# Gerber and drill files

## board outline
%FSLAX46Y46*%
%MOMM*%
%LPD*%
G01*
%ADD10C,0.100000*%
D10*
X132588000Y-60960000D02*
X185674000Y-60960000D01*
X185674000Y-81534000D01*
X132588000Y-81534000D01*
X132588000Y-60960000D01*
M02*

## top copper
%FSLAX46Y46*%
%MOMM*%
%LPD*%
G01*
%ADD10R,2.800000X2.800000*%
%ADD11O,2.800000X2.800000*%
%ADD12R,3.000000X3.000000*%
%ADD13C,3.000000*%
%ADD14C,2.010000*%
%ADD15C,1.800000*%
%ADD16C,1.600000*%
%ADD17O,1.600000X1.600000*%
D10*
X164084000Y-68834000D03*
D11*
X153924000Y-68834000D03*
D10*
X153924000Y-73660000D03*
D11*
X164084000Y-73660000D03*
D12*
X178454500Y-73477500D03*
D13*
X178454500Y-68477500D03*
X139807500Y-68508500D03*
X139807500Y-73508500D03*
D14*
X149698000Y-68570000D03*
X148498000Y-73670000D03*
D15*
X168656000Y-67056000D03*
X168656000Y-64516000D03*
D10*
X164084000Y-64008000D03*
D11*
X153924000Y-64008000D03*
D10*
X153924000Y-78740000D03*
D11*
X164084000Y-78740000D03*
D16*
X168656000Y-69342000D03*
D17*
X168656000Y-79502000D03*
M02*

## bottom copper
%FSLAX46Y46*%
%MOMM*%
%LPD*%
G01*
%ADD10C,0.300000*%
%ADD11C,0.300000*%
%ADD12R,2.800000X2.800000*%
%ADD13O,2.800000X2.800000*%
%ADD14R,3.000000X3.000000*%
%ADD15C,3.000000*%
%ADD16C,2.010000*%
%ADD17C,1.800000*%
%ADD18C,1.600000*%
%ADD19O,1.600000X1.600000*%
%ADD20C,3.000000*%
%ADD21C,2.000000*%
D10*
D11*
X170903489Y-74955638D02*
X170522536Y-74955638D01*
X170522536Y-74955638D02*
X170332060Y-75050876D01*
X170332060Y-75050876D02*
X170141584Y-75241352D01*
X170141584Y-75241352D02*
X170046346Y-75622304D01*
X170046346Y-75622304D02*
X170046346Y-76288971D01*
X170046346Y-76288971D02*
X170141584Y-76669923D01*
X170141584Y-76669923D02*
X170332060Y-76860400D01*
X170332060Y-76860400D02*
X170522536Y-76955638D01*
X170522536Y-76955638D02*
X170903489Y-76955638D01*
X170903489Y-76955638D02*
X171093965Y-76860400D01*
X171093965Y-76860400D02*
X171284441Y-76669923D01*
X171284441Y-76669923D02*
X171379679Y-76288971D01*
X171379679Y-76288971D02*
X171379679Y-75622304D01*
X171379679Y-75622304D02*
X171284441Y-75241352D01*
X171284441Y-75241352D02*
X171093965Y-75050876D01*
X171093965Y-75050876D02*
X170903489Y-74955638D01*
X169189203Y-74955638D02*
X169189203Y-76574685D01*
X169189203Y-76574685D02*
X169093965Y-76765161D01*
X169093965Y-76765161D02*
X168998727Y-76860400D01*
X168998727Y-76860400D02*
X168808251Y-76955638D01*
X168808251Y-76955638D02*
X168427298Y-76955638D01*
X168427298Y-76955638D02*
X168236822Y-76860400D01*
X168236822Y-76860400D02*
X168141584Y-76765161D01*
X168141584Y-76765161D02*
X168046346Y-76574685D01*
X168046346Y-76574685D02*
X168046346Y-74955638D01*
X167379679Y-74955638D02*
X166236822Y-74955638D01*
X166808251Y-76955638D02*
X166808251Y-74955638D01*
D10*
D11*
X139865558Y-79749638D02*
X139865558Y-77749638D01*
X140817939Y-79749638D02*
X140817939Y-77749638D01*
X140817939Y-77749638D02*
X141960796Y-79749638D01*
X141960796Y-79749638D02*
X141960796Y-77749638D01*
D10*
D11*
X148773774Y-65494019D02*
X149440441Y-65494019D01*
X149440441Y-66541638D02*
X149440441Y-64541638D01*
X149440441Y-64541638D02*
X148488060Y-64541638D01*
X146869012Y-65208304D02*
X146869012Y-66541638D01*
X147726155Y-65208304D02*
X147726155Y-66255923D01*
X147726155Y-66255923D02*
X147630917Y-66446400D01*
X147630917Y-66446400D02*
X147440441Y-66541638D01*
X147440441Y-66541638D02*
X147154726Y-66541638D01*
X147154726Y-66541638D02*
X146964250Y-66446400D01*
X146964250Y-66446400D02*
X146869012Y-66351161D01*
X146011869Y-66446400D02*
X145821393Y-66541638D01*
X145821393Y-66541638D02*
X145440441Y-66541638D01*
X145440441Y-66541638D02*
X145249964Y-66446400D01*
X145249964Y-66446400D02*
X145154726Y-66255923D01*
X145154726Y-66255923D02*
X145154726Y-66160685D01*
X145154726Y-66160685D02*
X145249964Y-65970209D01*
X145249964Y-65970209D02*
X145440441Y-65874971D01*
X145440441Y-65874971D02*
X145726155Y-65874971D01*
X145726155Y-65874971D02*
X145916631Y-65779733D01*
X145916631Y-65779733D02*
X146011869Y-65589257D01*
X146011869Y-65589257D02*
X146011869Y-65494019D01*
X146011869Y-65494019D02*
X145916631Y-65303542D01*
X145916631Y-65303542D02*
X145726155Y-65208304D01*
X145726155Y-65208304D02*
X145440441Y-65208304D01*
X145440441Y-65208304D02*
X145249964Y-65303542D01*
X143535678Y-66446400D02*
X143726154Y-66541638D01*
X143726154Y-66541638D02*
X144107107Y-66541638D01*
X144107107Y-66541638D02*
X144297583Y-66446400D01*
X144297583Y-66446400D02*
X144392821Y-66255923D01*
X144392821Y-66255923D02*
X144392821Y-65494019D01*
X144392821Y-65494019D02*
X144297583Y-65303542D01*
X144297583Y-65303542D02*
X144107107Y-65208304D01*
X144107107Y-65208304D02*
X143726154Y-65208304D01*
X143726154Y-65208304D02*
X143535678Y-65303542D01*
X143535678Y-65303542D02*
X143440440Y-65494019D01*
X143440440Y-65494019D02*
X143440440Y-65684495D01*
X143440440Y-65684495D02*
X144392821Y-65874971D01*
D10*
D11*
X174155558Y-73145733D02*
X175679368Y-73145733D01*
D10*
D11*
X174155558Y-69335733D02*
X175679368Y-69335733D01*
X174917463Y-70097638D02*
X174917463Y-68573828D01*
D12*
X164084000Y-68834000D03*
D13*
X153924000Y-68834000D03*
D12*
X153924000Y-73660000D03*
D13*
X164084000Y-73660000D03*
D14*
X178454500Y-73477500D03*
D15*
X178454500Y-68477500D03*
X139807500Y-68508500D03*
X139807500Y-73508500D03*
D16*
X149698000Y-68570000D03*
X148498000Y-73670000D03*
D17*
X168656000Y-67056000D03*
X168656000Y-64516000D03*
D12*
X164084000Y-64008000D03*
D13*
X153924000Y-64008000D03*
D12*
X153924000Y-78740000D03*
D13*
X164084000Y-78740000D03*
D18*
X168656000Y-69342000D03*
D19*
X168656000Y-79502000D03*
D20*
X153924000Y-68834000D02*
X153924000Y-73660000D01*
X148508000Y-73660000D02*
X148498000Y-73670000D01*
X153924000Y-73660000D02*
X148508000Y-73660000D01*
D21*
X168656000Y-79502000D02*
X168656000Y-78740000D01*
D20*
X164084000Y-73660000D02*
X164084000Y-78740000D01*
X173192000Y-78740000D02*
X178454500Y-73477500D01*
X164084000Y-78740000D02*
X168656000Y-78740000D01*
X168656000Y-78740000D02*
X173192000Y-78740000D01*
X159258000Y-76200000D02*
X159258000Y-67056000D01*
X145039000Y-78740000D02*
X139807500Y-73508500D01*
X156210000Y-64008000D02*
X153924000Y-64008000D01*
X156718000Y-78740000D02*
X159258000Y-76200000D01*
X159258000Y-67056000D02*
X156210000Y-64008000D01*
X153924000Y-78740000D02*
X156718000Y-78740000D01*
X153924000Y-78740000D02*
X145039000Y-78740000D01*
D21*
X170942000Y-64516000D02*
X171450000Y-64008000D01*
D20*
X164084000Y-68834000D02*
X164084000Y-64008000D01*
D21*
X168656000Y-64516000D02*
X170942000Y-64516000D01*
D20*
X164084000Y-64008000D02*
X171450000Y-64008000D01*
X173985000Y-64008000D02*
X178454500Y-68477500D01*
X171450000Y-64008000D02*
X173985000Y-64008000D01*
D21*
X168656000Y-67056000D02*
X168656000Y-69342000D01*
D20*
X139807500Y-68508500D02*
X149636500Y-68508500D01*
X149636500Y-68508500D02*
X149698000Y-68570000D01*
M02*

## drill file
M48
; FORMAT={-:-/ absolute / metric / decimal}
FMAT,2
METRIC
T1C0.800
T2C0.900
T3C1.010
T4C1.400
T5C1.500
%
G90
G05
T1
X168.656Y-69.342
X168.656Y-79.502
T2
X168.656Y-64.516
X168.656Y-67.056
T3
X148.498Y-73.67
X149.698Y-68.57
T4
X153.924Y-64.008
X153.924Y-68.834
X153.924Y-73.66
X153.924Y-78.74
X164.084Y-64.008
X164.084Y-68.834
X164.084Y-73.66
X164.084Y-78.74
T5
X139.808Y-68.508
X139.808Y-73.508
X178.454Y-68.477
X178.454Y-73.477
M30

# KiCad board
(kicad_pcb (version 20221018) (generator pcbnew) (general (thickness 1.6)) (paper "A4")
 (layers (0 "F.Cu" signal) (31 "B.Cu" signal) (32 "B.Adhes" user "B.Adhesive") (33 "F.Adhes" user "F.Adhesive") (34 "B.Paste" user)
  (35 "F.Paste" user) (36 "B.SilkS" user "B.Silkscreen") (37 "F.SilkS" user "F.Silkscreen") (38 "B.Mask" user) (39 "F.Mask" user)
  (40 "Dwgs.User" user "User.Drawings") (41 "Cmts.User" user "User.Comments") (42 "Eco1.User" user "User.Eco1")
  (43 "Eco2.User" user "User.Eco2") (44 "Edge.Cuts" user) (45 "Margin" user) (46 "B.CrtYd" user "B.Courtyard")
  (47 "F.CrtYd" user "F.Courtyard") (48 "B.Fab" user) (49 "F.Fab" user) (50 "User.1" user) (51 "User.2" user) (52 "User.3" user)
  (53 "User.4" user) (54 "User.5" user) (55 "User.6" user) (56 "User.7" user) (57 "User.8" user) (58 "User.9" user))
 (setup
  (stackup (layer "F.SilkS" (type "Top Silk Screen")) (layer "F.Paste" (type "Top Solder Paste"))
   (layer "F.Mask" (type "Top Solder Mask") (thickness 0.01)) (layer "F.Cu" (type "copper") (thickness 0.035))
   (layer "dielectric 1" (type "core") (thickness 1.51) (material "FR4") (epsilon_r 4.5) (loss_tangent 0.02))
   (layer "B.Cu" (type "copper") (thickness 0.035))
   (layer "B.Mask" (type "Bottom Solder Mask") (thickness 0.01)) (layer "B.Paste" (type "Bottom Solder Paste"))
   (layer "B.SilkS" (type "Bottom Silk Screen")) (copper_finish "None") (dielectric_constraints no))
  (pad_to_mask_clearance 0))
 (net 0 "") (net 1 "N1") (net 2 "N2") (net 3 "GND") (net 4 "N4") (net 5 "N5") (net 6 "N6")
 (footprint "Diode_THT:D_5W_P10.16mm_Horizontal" (layer "F.Cu") (at 164.084 68.834 180)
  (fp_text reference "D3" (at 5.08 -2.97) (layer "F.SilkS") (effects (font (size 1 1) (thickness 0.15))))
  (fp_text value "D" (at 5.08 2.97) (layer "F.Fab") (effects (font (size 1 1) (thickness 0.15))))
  (pad "1" thru_hole rect (at 0 0 180) (size 2.8 2.8) (drill 1.4) (layers "*.Cu" "*.Mask") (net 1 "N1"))
  (pad "2" thru_hole oval (at 10.16 0 180) (size 2.8 2.8) (drill 1.4) (layers "*.Cu" "*.Mask") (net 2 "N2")))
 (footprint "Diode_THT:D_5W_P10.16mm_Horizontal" (layer "F.Cu") (at 153.924 73.66)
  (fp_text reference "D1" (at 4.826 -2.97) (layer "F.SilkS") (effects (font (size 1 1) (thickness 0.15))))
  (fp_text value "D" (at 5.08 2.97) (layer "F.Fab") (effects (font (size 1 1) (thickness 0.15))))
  (pad "1" thru_hole rect (at 0 0) (size 2.8 2.8) (drill 1.4) (layers "*.Cu" "*.Mask") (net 2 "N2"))
  (pad "2" thru_hole oval (at 10.16 0) (size 2.8 2.8) (drill 1.4) (layers "*.Cu" "*.Mask") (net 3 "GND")))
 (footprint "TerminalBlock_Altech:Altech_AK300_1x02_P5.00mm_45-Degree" (layer "F.Cu") (at 178.4545 73.4775 90)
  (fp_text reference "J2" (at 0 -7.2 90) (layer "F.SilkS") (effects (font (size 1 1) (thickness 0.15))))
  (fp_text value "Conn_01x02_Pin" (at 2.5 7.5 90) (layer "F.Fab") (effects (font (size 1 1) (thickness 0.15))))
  (pad "1" thru_hole rect (at 0 0 90) (size 3 3) (drill 1.5) (layers "*.Cu" "*.Mask") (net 3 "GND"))
  (pad "2" thru_hole circle (at 5 0 90) (size 3 3) (drill 1.5) (layers "*.Cu" "*.Mask") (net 1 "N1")))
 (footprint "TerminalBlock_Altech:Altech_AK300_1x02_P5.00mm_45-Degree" (layer "F.Cu") (at 139.8075 68.5085 -90)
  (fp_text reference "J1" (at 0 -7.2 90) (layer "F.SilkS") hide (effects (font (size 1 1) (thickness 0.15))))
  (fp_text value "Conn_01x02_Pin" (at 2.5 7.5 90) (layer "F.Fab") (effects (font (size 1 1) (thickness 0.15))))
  (pad "1" thru_hole circle (at 0 0 270) (size 3 3) (drill 1.5) (layers "*.Cu" "*.Mask") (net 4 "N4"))
  (pad "2" thru_hole circle (at 5 0 270) (size 3 3) (drill 1.5) (layers "*.Cu" "*.Mask") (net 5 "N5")))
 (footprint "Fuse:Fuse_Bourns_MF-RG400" (layer "F.Cu") (at 149.698 68.57 -90)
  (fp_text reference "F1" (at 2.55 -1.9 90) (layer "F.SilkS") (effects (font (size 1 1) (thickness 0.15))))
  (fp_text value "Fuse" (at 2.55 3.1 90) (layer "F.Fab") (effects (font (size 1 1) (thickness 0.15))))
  (pad "1" thru_hole circle (at 0 0 270) (size 2.01 2.01) (drill 1.01) (layers "*.Cu" "*.Mask") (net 4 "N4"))
  (pad "2" thru_hole circle (at 5.1 1.2 270) (size 2.01 2.01) (drill 1.01) (layers "*.Cu" "*.Mask") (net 2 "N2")))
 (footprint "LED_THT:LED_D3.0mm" (layer "F.Cu") (at 168.656 67.056 90)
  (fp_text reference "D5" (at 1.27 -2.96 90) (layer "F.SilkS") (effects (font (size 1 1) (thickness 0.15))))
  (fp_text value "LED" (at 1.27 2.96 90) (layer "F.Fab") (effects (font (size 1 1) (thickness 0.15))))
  (pad "1" thru_hole circle (at 0 0 90) (size 1.8 1.8) (drill 0.9) (layers "*.Cu" "*.Mask") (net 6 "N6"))
  (pad "2" thru_hole circle (at 2.54 0 90) (size 1.8 1.8) (drill 0.9) (layers "*.Cu" "*.Mask") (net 1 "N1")))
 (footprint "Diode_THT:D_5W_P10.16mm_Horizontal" (layer "F.Cu") (at 164.084 64.008 180)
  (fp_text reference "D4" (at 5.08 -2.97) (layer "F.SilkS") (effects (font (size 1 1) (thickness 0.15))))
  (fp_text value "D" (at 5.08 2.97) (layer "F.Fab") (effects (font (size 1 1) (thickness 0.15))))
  (pad "1" thru_hole rect (at 0 0 180) (size 2.8 2.8) (drill 1.4) (layers "*.Cu" "*.Mask") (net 1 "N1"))
  (pad "2" thru_hole oval (at 10.16 0 180) (size 2.8 2.8) (drill 1.4) (layers "*.Cu" "*.Mask") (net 5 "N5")))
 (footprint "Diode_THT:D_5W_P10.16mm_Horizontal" (layer "F.Cu") (at 153.924 78.74)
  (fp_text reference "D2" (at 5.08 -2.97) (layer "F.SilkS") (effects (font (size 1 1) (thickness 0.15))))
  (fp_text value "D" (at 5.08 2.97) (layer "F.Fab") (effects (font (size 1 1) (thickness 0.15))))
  (pad "1" thru_hole rect (at 0 0) (size 2.8 2.8) (drill 1.4) (layers "*.Cu" "*.Mask") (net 5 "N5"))
  (pad "2" thru_hole oval (at 10.16 0) (size 2.8 2.8) (drill 1.4) (layers "*.Cu" "*.Mask") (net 3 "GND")))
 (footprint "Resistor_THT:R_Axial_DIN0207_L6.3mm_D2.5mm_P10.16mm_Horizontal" (layer "F.Cu") (at 168.656 69.342 -90)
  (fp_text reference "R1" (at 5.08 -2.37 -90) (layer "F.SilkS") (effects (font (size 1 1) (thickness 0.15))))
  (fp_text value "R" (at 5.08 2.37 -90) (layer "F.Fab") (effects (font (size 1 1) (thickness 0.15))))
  (pad "1" thru_hole circle (at 0 0 270) (size 1.6 1.6) (drill 0.8) (layers "*.Cu" "*.Mask") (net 6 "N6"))
  (pad "2" thru_hole oval (at 10.16 0 270) (size 1.6 1.6) (drill 0.8) (layers "*.Cu" "*.Mask") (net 3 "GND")))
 (gr_rect (start 132.588 60.96) (end 185.674 81.534) (stroke (width 0.1) (type default)) (fill none) (layer "Edge.Cuts"))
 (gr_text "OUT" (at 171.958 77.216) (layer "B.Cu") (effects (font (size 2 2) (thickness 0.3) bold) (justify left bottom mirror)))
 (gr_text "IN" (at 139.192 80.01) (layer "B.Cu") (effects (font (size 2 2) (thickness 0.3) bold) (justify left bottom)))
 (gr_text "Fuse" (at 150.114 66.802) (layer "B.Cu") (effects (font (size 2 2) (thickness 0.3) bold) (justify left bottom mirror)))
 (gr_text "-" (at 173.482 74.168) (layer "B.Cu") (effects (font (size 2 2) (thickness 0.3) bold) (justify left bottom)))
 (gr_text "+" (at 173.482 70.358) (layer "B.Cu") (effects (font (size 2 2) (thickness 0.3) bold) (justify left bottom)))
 (segment (start 153.924 68.834) (end 153.924 73.66) (width 3) (layer "B.Cu") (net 2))
 (segment (start 148.508 73.66) (end 148.498 73.67) (width 3) (layer "B.Cu") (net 2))
 (segment (start 153.924 73.66) (end 148.508 73.66) (width 3) (layer "B.Cu") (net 2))
 (segment (start 168.656 79.502) (end 168.656 78.74) (width 2) (layer "B.Cu") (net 3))
 (segment (start 164.084 73.66) (end 164.084 78.74) (width 3) (layer "B.Cu") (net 3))
 (segment (start 173.192 78.74) (end 178.4545 73.4775) (width 3) (layer "B.Cu") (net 3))
 (segment (start 164.084 78.74) (end 168.656 78.74) (width 3) (layer "B.Cu") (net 3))
 (segment (start 168.656 78.74) (end 173.192 78.74) (width 3) (layer "B.Cu") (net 3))
 (segment (start 159.258 76.2) (end 159.258 67.056) (width 3) (layer "B.Cu") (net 5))
 (segment (start 145.039 78.74) (end 139.8075 73.5085) (width 3) (layer "B.Cu") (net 5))
 (segment (start 156.21 64.008) (end 153.924 64.008) (width 3) (layer "B.Cu") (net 5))
 (segment (start 156.718 78.74) (end 159.258 76.2) (width 3) (layer "B.Cu") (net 5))
 (segment (start 159.258 67.056) (end 156.21 64.008) (width 3) (layer "B.Cu") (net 5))
 (segment (start 153.924 78.74) (end 156.718 78.74) (width 3) (layer "B.Cu") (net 5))
 (segment (start 153.924 78.74) (end 145.039 78.74) (width 3) (layer "B.Cu") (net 5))
 (segment (start 170.942 64.516) (end 171.45 64.008) (width 2) (layer "B.Cu") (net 1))
 (segment (start 164.084 68.834) (end 164.084 64.008) (width 3) (layer "B.Cu") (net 1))
 (segment (start 168.656 64.516) (end 170.942 64.516) (width 2) (layer "B.Cu") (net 1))
 (segment (start 164.084 64.008) (end 171.45 64.008) (width 3) (layer "B.Cu") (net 1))
 (segment (start 173.985 64.008) (end 178.4545 68.4775) (width 3) (layer "B.Cu") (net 1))
 (segment (start 171.45 64.008) (end 173.985 64.008) (width 3) (layer "B.Cu") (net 1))
 (segment (start 168.656 67.056) (end 168.656 69.342) (width 2) (layer "B.Cu") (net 6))
 (segment (start 139.8075 68.5085) (end 149.6365 68.5085) (width 3) (layer "B.Cu") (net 4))
 (segment (start 149.6365 68.5085) (end 149.698 68.57) (width 3) (layer "B.Cu") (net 4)))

